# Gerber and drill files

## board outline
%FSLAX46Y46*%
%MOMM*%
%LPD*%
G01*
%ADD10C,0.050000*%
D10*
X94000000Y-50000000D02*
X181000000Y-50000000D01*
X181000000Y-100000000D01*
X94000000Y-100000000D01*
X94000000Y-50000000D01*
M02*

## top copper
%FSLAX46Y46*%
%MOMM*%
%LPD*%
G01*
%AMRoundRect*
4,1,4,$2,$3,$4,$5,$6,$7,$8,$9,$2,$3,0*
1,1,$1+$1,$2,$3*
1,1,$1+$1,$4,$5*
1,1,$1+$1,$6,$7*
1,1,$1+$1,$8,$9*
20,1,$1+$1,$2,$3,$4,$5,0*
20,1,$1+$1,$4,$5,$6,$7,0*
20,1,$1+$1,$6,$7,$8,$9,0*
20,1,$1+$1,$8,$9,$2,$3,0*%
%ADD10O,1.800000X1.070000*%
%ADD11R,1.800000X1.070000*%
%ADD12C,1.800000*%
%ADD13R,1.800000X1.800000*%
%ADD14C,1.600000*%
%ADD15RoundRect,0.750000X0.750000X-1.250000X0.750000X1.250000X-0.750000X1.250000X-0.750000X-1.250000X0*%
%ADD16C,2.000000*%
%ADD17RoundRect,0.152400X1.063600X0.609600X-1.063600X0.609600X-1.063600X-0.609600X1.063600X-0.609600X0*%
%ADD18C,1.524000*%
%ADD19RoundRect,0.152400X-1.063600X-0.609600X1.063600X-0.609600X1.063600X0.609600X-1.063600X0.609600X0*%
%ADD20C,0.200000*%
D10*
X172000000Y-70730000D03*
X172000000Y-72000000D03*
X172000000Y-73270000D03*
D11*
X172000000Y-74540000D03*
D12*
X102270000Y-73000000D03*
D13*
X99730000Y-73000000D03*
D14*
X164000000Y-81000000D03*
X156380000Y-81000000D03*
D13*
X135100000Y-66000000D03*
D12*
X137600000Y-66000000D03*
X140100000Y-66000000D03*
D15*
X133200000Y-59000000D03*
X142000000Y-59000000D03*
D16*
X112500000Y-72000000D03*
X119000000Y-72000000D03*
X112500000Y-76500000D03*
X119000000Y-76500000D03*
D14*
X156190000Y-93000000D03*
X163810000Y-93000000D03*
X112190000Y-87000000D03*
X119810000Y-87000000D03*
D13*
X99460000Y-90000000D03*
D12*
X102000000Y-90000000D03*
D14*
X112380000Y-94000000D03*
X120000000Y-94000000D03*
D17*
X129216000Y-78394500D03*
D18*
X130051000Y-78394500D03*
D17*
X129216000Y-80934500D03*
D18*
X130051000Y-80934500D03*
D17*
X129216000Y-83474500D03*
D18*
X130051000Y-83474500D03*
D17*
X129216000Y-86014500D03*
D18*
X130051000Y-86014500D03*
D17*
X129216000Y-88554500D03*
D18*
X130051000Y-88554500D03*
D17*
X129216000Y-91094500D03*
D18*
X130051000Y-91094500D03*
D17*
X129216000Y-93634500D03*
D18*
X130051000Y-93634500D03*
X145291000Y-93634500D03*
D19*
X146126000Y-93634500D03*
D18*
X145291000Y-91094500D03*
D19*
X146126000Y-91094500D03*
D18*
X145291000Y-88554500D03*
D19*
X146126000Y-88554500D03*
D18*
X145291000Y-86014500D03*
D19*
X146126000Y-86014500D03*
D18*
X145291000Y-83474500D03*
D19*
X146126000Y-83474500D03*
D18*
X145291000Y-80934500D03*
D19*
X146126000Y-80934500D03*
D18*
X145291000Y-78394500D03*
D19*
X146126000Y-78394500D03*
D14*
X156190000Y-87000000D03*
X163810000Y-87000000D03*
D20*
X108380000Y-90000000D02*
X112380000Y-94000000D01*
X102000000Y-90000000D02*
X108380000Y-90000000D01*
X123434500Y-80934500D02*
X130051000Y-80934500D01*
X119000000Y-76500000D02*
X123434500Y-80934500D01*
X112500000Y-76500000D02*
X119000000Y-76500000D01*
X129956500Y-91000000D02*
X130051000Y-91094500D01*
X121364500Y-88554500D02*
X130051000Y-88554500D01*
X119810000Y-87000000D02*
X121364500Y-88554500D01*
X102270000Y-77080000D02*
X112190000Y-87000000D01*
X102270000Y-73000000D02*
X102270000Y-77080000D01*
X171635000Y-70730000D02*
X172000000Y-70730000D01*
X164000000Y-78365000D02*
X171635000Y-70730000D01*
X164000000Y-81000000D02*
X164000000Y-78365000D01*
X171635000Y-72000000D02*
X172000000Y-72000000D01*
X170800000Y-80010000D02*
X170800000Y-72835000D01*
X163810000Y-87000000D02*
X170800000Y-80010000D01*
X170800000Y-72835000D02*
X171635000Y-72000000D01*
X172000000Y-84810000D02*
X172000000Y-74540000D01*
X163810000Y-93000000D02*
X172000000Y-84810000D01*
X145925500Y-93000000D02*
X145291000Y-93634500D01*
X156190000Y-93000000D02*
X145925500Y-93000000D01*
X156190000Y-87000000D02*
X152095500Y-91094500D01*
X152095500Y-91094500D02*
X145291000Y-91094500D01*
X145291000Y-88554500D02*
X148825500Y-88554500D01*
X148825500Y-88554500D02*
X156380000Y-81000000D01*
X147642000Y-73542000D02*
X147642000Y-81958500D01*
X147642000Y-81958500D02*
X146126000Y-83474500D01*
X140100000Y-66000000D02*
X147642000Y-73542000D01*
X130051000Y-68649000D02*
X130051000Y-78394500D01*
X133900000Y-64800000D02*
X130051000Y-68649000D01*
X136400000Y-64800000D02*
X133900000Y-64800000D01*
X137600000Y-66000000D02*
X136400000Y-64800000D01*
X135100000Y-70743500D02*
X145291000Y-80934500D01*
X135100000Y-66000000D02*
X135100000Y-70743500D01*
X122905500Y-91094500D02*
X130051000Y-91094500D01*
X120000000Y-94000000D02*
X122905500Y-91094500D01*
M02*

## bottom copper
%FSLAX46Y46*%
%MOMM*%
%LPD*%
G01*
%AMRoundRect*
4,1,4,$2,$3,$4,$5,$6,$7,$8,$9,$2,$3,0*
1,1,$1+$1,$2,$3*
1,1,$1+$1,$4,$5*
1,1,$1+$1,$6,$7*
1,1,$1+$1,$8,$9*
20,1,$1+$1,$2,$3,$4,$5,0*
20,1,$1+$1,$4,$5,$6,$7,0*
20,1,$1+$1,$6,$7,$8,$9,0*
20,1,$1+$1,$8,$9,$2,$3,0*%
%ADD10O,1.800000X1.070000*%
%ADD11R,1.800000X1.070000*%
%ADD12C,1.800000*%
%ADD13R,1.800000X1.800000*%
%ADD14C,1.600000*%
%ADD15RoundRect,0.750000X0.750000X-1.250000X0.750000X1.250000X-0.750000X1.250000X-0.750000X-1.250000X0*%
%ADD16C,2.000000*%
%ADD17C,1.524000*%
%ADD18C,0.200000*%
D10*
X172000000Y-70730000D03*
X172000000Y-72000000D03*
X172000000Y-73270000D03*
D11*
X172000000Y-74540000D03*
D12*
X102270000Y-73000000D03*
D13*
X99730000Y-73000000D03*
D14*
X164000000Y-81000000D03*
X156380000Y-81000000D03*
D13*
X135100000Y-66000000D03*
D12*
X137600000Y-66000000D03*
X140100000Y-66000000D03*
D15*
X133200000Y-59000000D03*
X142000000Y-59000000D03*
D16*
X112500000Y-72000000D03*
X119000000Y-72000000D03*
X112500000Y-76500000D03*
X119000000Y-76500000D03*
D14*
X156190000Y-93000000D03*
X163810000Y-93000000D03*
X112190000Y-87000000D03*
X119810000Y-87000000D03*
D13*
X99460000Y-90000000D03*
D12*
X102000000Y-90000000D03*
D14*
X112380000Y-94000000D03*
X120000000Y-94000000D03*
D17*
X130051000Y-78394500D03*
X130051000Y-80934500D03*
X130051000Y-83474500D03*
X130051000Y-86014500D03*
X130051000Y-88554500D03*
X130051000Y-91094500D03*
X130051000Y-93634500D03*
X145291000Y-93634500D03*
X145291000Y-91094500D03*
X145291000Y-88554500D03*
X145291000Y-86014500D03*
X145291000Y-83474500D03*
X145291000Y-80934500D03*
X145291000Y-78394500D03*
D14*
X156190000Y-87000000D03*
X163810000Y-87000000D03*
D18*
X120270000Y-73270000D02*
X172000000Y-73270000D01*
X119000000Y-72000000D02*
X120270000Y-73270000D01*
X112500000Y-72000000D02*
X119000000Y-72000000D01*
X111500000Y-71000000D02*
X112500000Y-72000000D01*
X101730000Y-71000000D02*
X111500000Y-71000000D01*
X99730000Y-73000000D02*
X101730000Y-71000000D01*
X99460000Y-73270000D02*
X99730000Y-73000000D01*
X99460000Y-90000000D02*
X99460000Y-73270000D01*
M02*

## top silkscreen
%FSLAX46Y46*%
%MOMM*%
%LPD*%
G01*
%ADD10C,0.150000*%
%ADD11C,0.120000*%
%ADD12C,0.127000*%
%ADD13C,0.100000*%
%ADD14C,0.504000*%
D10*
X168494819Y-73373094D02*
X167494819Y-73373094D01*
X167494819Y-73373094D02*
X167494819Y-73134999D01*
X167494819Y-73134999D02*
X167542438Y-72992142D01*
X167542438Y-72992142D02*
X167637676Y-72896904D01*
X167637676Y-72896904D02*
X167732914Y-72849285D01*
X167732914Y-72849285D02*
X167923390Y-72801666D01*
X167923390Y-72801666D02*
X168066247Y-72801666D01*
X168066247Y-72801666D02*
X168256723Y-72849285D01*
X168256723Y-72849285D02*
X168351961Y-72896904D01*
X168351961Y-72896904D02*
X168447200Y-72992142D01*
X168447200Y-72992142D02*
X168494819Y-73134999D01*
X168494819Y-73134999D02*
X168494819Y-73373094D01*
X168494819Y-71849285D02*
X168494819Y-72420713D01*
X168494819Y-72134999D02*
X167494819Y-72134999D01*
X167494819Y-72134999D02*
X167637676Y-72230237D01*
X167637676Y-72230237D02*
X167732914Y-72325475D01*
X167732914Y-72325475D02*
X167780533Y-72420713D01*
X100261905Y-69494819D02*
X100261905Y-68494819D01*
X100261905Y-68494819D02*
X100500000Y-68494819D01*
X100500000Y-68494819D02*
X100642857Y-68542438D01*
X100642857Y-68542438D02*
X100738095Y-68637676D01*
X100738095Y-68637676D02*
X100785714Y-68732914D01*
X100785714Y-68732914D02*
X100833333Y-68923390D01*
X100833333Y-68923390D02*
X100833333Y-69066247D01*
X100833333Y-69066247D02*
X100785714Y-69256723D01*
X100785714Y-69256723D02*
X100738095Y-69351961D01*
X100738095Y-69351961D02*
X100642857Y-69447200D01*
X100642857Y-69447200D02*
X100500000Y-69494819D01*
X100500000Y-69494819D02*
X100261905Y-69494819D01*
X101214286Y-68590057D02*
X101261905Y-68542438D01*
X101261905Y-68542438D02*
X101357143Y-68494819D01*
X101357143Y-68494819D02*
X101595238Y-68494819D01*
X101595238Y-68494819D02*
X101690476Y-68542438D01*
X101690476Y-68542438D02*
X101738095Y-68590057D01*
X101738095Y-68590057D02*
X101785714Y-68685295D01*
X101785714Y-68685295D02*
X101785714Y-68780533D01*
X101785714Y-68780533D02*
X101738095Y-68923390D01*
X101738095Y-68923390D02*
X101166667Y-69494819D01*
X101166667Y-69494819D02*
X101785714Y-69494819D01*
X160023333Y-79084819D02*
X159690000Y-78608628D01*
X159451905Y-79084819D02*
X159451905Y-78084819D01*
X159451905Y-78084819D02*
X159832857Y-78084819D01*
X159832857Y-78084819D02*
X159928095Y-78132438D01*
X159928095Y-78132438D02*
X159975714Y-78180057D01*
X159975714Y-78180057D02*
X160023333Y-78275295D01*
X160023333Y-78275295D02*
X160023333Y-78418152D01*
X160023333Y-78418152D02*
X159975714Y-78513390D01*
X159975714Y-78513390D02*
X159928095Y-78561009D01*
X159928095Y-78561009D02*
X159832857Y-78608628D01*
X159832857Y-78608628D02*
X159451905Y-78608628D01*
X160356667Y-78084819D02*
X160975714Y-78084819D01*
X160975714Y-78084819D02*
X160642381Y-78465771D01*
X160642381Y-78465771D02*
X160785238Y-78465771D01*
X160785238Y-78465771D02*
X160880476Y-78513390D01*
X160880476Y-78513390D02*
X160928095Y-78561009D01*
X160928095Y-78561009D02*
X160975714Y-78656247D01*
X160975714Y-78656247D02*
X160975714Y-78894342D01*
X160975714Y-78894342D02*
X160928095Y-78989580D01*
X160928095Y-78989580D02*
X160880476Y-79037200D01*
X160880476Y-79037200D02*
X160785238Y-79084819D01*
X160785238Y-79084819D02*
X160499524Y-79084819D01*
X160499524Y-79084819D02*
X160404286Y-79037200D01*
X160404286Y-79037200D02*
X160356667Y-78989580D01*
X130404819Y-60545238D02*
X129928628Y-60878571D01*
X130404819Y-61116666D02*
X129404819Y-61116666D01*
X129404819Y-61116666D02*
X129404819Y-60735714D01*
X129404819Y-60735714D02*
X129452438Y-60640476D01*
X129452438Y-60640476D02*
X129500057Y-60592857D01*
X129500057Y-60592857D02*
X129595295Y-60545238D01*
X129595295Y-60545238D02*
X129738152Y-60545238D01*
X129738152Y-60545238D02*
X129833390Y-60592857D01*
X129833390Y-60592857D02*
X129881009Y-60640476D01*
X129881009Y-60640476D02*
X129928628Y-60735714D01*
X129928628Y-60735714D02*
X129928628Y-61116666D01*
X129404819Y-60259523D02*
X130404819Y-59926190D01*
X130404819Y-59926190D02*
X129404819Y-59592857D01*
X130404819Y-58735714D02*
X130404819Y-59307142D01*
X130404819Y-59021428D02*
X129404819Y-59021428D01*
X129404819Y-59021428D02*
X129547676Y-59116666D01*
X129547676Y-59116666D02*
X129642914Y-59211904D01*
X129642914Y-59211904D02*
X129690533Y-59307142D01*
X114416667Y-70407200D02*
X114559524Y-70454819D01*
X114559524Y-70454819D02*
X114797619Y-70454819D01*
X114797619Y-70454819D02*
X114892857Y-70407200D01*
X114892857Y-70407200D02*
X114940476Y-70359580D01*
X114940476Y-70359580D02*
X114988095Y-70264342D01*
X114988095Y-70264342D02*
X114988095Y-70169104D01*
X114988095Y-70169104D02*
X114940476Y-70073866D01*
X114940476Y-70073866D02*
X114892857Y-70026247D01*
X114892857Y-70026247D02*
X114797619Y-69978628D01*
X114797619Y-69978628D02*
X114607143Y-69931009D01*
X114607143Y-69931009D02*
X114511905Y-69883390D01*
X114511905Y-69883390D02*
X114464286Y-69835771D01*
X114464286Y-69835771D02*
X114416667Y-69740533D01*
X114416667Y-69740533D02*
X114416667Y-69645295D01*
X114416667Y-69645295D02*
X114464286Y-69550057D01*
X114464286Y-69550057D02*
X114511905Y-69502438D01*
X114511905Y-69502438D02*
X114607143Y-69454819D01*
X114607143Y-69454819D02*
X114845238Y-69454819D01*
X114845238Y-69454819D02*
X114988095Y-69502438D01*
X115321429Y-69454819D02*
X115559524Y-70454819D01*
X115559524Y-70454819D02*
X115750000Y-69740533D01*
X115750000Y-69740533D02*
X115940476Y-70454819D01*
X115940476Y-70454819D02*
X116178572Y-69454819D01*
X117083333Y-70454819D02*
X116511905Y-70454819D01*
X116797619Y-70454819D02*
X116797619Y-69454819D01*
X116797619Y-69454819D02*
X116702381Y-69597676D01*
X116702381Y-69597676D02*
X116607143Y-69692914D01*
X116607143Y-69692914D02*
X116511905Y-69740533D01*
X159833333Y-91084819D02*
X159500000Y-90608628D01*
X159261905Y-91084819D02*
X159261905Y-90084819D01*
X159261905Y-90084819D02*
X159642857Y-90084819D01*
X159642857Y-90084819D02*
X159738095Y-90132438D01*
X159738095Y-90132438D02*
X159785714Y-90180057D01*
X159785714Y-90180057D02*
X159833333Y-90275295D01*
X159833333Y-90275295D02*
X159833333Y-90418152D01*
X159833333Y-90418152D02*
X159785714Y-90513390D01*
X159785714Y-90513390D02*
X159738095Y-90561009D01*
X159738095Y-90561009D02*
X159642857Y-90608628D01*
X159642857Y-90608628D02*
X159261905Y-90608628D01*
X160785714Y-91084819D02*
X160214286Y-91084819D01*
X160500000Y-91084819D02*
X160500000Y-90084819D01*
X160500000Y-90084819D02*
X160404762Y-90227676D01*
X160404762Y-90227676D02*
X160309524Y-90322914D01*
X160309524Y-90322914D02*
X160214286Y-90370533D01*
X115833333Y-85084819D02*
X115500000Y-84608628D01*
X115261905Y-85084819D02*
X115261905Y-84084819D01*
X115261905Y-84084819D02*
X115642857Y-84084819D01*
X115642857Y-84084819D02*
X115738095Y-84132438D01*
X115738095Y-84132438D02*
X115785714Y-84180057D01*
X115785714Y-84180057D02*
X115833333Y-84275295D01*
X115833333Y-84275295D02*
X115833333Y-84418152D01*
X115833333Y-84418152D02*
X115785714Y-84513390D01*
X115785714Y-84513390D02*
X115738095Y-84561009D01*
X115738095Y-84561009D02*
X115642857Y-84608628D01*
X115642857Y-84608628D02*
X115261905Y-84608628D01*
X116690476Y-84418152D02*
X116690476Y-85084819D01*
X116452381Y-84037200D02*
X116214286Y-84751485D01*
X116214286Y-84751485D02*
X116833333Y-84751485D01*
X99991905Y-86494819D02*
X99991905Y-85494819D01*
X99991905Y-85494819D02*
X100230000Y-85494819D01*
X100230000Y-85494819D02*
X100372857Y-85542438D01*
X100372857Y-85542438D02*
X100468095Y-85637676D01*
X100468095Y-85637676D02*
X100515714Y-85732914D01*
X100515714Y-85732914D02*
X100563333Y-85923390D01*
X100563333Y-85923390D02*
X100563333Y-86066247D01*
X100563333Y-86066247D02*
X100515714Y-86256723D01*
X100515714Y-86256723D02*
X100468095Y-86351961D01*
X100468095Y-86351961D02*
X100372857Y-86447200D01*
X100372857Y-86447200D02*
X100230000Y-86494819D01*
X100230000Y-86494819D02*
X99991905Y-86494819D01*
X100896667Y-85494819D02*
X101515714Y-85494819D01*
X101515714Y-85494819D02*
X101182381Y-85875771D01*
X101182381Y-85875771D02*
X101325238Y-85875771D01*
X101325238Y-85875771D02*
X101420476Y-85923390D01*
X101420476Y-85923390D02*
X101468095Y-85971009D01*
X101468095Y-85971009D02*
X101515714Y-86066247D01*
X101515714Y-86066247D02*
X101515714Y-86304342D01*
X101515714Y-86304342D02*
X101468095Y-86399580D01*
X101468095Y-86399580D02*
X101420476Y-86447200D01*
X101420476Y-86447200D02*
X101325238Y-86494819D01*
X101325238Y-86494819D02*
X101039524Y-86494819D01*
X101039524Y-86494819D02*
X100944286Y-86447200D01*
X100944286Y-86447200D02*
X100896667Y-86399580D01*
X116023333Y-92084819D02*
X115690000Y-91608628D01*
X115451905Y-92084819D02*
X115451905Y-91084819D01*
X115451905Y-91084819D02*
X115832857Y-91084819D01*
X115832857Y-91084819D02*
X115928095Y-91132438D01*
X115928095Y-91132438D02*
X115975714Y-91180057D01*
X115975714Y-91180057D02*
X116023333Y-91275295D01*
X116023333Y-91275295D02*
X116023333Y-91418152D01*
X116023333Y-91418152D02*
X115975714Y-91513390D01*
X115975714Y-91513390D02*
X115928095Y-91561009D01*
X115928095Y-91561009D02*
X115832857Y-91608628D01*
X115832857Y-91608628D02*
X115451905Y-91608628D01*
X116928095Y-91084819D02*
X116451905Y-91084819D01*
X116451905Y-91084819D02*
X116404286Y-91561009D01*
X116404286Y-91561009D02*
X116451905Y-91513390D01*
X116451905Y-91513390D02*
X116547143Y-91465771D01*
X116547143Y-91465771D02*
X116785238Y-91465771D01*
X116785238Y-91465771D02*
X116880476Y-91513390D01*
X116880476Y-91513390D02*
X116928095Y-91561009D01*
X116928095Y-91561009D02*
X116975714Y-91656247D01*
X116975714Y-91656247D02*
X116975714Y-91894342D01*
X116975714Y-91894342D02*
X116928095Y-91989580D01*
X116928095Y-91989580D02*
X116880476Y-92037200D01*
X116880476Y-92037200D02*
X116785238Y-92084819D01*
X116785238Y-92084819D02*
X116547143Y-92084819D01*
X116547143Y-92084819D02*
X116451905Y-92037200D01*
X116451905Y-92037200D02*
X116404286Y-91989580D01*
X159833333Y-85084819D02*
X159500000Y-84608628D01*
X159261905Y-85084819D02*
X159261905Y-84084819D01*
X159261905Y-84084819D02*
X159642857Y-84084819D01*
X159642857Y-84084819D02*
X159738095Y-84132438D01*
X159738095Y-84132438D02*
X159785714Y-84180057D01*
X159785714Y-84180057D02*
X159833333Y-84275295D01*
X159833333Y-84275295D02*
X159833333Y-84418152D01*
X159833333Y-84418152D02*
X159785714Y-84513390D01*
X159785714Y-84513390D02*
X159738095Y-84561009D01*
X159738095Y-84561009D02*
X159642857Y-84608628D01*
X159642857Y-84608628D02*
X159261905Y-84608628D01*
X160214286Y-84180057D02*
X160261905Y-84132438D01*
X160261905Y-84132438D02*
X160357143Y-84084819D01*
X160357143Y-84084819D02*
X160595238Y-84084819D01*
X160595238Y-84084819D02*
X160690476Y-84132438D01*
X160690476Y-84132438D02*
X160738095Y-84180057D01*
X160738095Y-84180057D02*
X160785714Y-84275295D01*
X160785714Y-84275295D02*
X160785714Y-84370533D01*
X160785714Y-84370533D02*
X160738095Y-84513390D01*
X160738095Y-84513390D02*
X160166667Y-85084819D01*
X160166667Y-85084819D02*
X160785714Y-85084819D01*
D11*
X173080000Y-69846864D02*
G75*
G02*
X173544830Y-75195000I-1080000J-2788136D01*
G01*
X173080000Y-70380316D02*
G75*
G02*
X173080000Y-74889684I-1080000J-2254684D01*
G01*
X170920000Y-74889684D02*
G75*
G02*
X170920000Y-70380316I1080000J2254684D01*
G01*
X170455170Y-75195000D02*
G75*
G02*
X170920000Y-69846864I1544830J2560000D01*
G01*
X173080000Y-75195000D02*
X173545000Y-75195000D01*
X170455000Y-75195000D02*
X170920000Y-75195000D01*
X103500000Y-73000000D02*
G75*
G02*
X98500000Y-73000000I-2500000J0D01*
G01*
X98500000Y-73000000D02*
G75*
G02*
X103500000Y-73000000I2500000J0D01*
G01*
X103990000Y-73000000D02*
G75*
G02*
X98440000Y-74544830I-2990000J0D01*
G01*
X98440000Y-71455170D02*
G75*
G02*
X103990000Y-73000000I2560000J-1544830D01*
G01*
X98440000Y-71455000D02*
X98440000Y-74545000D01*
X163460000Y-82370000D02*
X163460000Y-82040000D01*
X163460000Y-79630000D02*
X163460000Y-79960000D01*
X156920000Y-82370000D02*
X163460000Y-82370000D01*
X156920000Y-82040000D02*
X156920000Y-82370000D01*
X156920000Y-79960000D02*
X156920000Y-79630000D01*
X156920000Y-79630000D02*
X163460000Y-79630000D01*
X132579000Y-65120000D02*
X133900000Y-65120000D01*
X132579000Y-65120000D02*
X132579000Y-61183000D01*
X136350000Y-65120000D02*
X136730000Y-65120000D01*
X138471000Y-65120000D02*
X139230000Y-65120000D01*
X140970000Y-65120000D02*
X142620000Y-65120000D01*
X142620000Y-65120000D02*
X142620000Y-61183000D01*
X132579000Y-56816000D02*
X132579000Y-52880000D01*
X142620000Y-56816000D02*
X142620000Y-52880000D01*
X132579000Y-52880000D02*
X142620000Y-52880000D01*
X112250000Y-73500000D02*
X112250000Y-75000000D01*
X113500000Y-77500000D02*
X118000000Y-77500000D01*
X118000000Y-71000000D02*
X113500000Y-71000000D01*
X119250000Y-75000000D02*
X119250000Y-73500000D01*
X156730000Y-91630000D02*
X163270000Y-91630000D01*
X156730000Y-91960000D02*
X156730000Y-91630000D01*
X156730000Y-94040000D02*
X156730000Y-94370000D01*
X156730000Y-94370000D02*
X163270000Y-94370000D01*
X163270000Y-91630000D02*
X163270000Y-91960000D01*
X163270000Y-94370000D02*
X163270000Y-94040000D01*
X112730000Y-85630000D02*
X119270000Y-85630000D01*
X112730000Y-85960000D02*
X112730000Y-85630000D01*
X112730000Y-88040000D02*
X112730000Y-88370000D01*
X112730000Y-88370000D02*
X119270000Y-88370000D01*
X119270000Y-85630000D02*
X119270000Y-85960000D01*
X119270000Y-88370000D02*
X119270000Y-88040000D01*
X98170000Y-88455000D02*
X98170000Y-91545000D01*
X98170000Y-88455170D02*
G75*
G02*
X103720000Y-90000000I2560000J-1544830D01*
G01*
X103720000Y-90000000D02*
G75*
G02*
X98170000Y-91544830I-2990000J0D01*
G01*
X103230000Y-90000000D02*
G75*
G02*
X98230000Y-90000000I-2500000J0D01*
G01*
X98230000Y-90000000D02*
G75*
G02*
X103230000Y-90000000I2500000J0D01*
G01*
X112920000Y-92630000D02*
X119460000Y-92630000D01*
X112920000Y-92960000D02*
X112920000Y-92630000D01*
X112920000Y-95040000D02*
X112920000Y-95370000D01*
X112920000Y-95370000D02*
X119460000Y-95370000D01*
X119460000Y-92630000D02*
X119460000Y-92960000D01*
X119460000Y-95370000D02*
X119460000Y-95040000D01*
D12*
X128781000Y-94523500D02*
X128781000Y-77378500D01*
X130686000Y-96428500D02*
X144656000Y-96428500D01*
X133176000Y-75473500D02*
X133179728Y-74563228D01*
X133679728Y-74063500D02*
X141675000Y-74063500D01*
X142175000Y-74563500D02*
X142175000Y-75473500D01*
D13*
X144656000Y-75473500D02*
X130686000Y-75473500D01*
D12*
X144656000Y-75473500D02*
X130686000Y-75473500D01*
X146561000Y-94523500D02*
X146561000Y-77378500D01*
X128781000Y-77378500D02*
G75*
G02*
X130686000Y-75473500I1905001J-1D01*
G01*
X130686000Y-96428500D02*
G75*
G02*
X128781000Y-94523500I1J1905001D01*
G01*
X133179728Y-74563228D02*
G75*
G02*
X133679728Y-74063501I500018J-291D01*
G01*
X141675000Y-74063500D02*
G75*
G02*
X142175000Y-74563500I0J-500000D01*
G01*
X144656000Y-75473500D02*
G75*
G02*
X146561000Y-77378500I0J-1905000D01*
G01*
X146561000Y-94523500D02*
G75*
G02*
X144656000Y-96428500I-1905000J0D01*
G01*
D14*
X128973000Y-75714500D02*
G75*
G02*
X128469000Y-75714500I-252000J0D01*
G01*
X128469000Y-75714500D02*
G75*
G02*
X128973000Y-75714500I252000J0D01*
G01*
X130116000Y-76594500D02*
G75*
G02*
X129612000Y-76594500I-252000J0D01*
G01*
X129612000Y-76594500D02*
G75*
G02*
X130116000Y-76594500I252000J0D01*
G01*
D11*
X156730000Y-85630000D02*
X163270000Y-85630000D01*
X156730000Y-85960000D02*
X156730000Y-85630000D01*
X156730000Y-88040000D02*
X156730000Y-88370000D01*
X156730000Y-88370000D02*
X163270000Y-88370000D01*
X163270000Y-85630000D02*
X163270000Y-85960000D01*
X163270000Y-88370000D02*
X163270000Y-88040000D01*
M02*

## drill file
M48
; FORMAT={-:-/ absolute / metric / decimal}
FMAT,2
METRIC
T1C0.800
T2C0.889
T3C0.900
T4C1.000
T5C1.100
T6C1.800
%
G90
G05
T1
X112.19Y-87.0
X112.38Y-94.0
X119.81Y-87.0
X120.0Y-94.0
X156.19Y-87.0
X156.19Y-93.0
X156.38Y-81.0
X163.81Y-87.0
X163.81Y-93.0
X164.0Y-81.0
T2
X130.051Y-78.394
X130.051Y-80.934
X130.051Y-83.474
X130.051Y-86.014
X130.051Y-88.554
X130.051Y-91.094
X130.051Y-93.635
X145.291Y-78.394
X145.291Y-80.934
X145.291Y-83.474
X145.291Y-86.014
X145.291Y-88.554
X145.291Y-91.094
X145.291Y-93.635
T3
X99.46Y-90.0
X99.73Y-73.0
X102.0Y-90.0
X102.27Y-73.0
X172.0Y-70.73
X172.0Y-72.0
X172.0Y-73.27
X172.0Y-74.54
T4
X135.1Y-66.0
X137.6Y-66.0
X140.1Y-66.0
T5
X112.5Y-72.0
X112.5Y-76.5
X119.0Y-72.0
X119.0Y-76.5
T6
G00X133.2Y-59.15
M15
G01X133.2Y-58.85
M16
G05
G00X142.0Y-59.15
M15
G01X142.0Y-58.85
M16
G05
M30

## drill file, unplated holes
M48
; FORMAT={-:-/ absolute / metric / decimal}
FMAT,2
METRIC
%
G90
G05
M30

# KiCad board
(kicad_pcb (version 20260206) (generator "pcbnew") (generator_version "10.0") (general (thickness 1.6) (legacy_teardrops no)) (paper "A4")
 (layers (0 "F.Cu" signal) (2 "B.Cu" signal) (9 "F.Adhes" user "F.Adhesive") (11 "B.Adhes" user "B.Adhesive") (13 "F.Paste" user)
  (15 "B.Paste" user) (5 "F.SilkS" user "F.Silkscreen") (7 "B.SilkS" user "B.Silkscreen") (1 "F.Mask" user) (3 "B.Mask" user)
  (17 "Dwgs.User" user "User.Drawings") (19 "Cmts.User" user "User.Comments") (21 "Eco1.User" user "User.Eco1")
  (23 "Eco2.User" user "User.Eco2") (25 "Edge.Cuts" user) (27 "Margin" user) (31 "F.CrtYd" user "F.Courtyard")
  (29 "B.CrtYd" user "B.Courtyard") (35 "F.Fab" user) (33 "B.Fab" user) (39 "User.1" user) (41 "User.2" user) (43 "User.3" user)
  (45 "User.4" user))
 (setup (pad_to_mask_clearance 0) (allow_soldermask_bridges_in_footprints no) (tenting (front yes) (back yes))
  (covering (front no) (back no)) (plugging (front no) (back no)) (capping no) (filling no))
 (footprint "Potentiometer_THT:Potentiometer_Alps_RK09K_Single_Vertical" (layer "F.Cu") (at 135.1 66 90)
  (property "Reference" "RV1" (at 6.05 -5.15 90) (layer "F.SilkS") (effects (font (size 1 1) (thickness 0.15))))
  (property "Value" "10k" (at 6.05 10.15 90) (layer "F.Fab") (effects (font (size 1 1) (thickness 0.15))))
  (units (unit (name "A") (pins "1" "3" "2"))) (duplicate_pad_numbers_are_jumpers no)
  (fp_line (start 13.12 -2.521) (end 13.12 7.52) (stroke (width 0.12) (type solid)) (layer "F.SilkS"))
  (fp_line (start 9.184 -2.521) (end 13.12 -2.521) (stroke (width 0.12) (type solid)) (layer "F.SilkS"))
  (fp_line (start 0.88 -2.521) (end 4.817 -2.521) (stroke (width 0.12) (type solid)) (layer "F.SilkS"))
  (fp_line (start 0.88 -2.521) (end 0.88 -1.2) (stroke (width 0.12) (type solid)) (layer "F.SilkS"))
  (fp_line (start 0.88 1.25) (end 0.88 1.63) (stroke (width 0.12) (type solid)) (layer "F.SilkS"))
  (fp_line (start 0.88 3.371) (end 0.88 4.13) (stroke (width 0.12) (type solid)) (layer "F.SilkS"))
  (fp_line (start 0.88 5.87) (end 0.88 7.52) (stroke (width 0.12) (type solid)) (layer "F.SilkS"))
  (fp_line (start 9.184 7.52) (end 13.12 7.52) (stroke (width 0.12) (type solid)) (layer "F.SilkS"))
  (fp_line (start 0.88 7.52) (end 4.817 7.52) (stroke (width 0.12) (type solid)) (layer "F.SilkS"))
  (pad "1" thru_hole rect (at 0 0 90) (size 1.8 1.8) (drill 1) (layers "*.Cu" "*.Mask") (remove_unused_layers no) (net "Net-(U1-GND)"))
  (pad "2" thru_hole circle (at 0 2.5 90) (size 1.8 1.8) (drill 1) (layers "*.Cu" "*.Mask") (remove_unused_layers no)
   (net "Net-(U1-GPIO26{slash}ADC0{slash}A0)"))
  (pad "3" thru_hole circle (at 0 5 90) (size 1.8 1.8) (drill 1) (layers "*.Cu" "*.Mask") (remove_unused_layers no) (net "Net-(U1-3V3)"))
  (pad "MP" thru_hole roundrect (at 7 -1.9 90) (size 4 3) (drill oval 2.1 1.8) (layers "*.Cu" "*.Mask") (remove_unused_layers no)
   (roundrect_rratio 0.25))
  (pad "MP" thru_hole roundrect (at 7 6.9 90) (size 4 3) (drill oval 2.1 1.8) (layers "*.Cu" "*.Mask") (remove_unused_layers no)
   (roundrect_rratio 0.25)))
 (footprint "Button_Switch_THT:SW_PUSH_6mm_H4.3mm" (layer "F.Cu") (at 112.5 72)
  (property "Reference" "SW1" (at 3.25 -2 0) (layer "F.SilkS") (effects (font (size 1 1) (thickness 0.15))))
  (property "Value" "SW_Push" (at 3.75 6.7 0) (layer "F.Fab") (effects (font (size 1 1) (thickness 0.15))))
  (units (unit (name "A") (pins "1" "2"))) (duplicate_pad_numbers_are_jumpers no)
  (fp_line (start -0.25 1.5) (end -0.25 3) (stroke (width 0.12) (type solid)) (layer "F.SilkS"))
  (fp_line (start 1 5.5) (end 5.5 5.5) (stroke (width 0.12) (type solid)) (layer "F.SilkS"))
  (fp_line (start 5.5 -1) (end 1 -1) (stroke (width 0.12) (type solid)) (layer "F.SilkS"))
  (fp_line (start 6.75 3) (end 6.75 1.5) (stroke (width 0.12) (type solid)) (layer "F.SilkS"))
  (pad "1" thru_hole circle (at 0 0 90) (size 2 2) (drill 1.1) (layers "*.Cu" "*.Mask") (remove_unused_layers no) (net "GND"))
  (pad "1" thru_hole circle (at 6.5 0 90) (size 2 2) (drill 1.1) (layers "*.Cu" "*.Mask") (remove_unused_layers no) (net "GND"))
  (pad "2" thru_hole circle (at 0 4.5 90) (size 2 2) (drill 1.1) (layers "*.Cu" "*.Mask") (remove_unused_layers no)
   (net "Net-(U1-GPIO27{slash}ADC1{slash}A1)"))
  (pad "2" thru_hole circle (at 6.5 4.5 90) (size 2 2) (drill 1.1) (layers "*.Cu" "*.Mask") (remove_unused_layers no)
   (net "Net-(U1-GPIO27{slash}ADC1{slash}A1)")))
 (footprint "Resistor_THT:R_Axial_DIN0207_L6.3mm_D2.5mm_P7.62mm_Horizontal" (layer "F.Cu") (at 156.38 81)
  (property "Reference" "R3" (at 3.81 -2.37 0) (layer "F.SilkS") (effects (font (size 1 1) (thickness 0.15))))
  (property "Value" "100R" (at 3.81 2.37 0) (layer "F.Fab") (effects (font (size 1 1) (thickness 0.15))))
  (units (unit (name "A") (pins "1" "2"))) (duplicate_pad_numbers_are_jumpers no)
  (fp_line (start 0.54 -1.37) (end 7.08 -1.37) (stroke (width 0.12) (type solid)) (layer "F.SilkS"))
  (fp_line (start 0.54 -1.04) (end 0.54 -1.37) (stroke (width 0.12) (type solid)) (layer "F.SilkS"))
  (fp_line (start 0.54 1.04) (end 0.54 1.37) (stroke (width 0.12) (type solid)) (layer "F.SilkS"))
  (fp_line (start 0.54 1.37) (end 7.08 1.37) (stroke (width 0.12) (type solid)) (layer "F.SilkS"))
  (fp_line (start 7.08 -1.37) (end 7.08 -1.04) (stroke (width 0.12) (type solid)) (layer "F.SilkS"))
  (fp_line (start 7.08 1.37) (end 7.08 1.04) (stroke (width 0.12) (type solid)) (layer "F.SilkS"))
  (pad "1" thru_hole circle (at 0 0) (size 1.6 1.6) (drill 0.8) (layers "*.Cu" "*.Mask") (remove_unused_layers no)
   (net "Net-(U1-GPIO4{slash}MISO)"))
  (pad "2" thru_hole circle (at 7.62 0) (size 1.6 1.6) (drill 0.8) (layers "*.Cu" "*.Mask") (remove_unused_layers no) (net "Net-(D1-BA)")))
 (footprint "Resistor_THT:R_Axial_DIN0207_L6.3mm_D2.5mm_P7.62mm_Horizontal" (layer "F.Cu") (at 156.19 93)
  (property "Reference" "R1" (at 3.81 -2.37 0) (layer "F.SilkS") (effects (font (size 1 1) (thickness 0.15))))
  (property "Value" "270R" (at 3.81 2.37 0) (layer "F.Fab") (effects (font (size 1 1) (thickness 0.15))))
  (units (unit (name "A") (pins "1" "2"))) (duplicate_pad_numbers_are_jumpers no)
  (fp_line (start 0.54 -1.37) (end 7.08 -1.37) (stroke (width 0.12) (type solid)) (layer "F.SilkS"))
  (fp_line (start 0.54 -1.04) (end 0.54 -1.37) (stroke (width 0.12) (type solid)) (layer "F.SilkS"))
  (fp_line (start 0.54 1.04) (end 0.54 1.37) (stroke (width 0.12) (type solid)) (layer "F.SilkS"))
  (fp_line (start 0.54 1.37) (end 7.08 1.37) (stroke (width 0.12) (type solid)) (layer "F.SilkS"))
  (fp_line (start 7.08 -1.37) (end 7.08 -1.04) (stroke (width 0.12) (type solid)) (layer "F.SilkS"))
  (fp_line (start 7.08 1.37) (end 7.08 1.04) (stroke (width 0.12) (type solid)) (layer "F.SilkS"))
  (pad "1" thru_hole circle (at 0 0) (size 1.6 1.6) (drill 0.8) (layers "*.Cu" "*.Mask") (remove_unused_layers no)
   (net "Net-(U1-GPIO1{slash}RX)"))
  (pad "2" thru_hole circle (at 7.62 0) (size 1.6 1.6) (drill 0.8) (layers "*.Cu" "*.Mask") (remove_unused_layers no) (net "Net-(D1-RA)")))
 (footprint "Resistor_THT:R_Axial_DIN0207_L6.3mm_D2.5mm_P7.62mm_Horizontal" (layer "F.Cu") (at 112.19 87)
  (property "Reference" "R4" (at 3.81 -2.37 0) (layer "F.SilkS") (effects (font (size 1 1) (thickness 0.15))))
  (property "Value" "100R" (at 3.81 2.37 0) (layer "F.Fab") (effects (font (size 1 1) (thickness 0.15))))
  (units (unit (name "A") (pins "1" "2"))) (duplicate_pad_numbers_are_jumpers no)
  (fp_line (start 0.54 -1.37) (end 7.08 -1.37) (stroke (width 0.12) (type solid)) (layer "F.SilkS"))
  (fp_line (start 0.54 -1.04) (end 0.54 -1.37) (stroke (width 0.12) (type solid)) (layer "F.SilkS"))
  (fp_line (start 0.54 1.04) (end 0.54 1.37) (stroke (width 0.12) (type solid)) (layer "F.SilkS"))
  (fp_line (start 0.54 1.37) (end 7.08 1.37) (stroke (width 0.12) (type solid)) (layer "F.SilkS"))
  (fp_line (start 7.08 -1.37) (end 7.08 -1.04) (stroke (width 0.12) (type solid)) (layer "F.SilkS"))
  (fp_line (start 7.08 1.37) (end 7.08 1.04) (stroke (width 0.12) (type solid)) (layer "F.SilkS"))
  (pad "1" thru_hole circle (at 0 0) (size 1.6 1.6) (drill 0.8) (layers "*.Cu" "*.Mask") (remove_unused_layers no) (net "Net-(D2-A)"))
  (pad "2" thru_hole circle (at 7.62 0) (size 1.6 1.6) (drill 0.8) (layers "*.Cu" "*.Mask") (remove_unused_layers no)
   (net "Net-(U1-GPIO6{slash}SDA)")))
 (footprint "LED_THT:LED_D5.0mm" (layer "F.Cu") (at 99.46 90)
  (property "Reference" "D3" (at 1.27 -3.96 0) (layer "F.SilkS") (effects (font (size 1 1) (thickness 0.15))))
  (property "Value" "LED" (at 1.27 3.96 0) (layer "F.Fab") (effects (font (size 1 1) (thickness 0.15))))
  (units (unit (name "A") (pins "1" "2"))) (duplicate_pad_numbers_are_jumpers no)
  (fp_line (start -1.29 -1.545) (end -1.29 1.545) (stroke (width 0.12) (type solid)) (layer "F.SilkS"))
  (fp_arc (start -1.29 -1.54483) (mid 2.071779 -2.880495) (end 4.26 0) (stroke (width 0.12) (type solid)) (layer "F.SilkS"))
  (fp_arc (start 4.26 0) (mid 2.071779 2.880495) (end -1.29 1.54483) (stroke (width 0.12) (type solid)) (layer "F.SilkS"))
  (fp_circle (center 1.27 0) (end 3.77 0) (stroke (width 0.12) (type solid)) (fill no) (layer "F.SilkS"))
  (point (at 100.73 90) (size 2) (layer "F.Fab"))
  (pad "1" thru_hole rect (at 0 0) (size 1.8 1.8) (drill 0.9) (layers "*.Cu" "*.Mask") (remove_unused_layers no) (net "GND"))
  (pad "2" thru_hole circle (at 2.54 0) (size 1.8 1.8) (drill 0.9) (layers "*.Cu" "*.Mask") (remove_unused_layers no) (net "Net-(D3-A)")))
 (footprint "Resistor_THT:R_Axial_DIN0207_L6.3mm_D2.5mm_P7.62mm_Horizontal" (layer "F.Cu") (at 112.38 94)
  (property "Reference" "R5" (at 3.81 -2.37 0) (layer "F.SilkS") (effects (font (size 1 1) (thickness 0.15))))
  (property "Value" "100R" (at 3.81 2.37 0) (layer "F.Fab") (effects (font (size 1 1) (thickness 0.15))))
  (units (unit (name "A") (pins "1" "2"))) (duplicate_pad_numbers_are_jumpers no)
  (fp_line (start 0.54 -1.37) (end 7.08 -1.37) (stroke (width 0.12) (type solid)) (layer "F.SilkS"))
  (fp_line (start 0.54 -1.04) (end 0.54 -1.37) (stroke (width 0.12) (type solid)) (layer "F.SilkS"))
  (fp_line (start 0.54 1.04) (end 0.54 1.37) (stroke (width 0.12) (type solid)) (layer "F.SilkS"))
  (fp_line (start 0.54 1.37) (end 7.08 1.37) (stroke (width 0.12) (type solid)) (layer "F.SilkS"))
  (fp_line (start 7.08 -1.37) (end 7.08 -1.04) (stroke (width 0.12) (type solid)) (layer "F.SilkS"))
  (fp_line (start 7.08 1.37) (end 7.08 1.04) (stroke (width 0.12) (type solid)) (layer "F.SilkS"))
  (pad "1" thru_hole circle (at 0 0) (size 1.6 1.6) (drill 0.8) (layers "*.Cu" "*.Mask") (remove_unused_layers no) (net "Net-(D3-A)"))
  (pad "2" thru_hole circle (at 7.62 0) (size 1.6 1.6) (drill 0.8) (layers "*.Cu" "*.Mask") (remove_unused_layers no)
   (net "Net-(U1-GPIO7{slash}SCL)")))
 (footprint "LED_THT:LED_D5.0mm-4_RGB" (layer "F.Cu") (at 172 74.54 90)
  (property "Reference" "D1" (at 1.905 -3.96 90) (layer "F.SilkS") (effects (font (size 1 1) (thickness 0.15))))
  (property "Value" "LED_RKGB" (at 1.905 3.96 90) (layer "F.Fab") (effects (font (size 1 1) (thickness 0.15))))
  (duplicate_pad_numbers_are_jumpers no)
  (fp_line (start -0.655 -1.545) (end -0.655 -1.08) (stroke (width 0.12) (type solid)) (layer "F.SilkS"))
  (fp_line (start -0.655 1.08) (end -0.655 1.545) (stroke (width 0.12) (type solid)) (layer "F.SilkS"))
  (fp_arc (start -0.655 -1.54483) (mid 2.163898 -2.97877) (end 4.693136 -1.08) (stroke (width 0.12) (type solid)) (layer "F.SilkS"))
  (fp_arc (start -0.349684 -1.08) (mid 1.905 -2.5) (end 4.159684 -1.08) (stroke (width 0.12) (type solid)) (layer "F.SilkS"))
  (fp_arc (start 4.693136 1.08) (mid 2.163898 2.97877) (end -0.655 1.54483) (stroke (width 0.12) (type solid)) (layer "F.SilkS"))
  (fp_arc (start 4.159684 1.08) (mid 1.905 2.5) (end -0.349684 1.08) (stroke (width 0.12) (type solid)) (layer "F.SilkS"))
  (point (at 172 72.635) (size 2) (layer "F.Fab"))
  (pad "1" thru_hole rect (at 0 0 90) (size 1.07 1.8) (drill 0.9) (layers "*.Cu" "*.Mask") (remove_unused_layers no) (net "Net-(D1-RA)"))
  (pad "2" thru_hole oval (at 1.27 0 90) (size 1.07 1.8) (drill 0.9) (layers "*.Cu" "*.Mask") (remove_unused_layers no) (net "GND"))
  (pad "3" thru_hole oval (at 2.54 0 90) (size 1.07 1.8) (drill 0.9) (layers "*.Cu" "*.Mask") (remove_unused_layers no) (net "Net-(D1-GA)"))
  (pad "4" thru_hole oval (at 3.81 0 90) (size 1.07 1.8) (drill 0.9) (layers "*.Cu" "*.Mask") (remove_unused_layers no) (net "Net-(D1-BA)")))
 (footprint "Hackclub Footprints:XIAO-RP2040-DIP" (layer "F.Cu") (at 137.671 86.0145)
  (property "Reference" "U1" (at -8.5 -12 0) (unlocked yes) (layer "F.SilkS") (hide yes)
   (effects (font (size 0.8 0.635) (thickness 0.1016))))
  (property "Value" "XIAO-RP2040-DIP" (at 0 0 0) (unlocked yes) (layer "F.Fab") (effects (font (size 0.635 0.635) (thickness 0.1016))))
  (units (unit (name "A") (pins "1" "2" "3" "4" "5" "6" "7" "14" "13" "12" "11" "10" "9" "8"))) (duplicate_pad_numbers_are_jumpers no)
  (fp_line (start -8.89 8.509) (end -8.89 -8.636) (stroke (width 0.127) (type solid)) (layer "F.SilkS"))
  (fp_line (start -6.985 10.414) (end 6.985 10.414) (stroke (width 0.127) (type solid)) (layer "F.SilkS"))
  (fp_line (start -4.495 -10.541) (end -4.491272 -11.451272) (stroke (width 0.127) (type solid)) (layer "F.SilkS"))
  (fp_line (start -3.991272 -11.951) (end 4.004 -11.951) (stroke (width 0.127) (type solid)) (layer "F.SilkS"))
  (fp_line (start 4.504 -11.451) (end 4.504 -10.541) (stroke (width 0.127) (type solid)) (layer "F.SilkS"))
  (fp_line (start 6.985 -10.541) (end -6.985 -10.541) (stroke (width 0.1) (type solid)) (layer "F.SilkS"))
  (fp_line (start 6.985 -10.541) (end -6.985 -10.541) (stroke (width 0.127) (type solid)) (layer "F.SilkS"))
  (fp_line (start 8.89 8.509) (end 8.89 -8.636) (stroke (width 0.127) (type solid)) (layer "F.SilkS"))
  (fp_arc (start -8.89 -8.636) (mid -8.332038 -9.983038) (end -6.985 -10.541) (stroke (width 0.127) (type solid)) (layer "F.SilkS"))
  (fp_arc (start -6.985 10.414) (mid -8.332038 9.856038) (end -8.89 8.509) (stroke (width 0.127) (type solid)) (layer "F.SilkS"))
  (fp_arc (start -4.491272 -11.451272) (mid -4.344728 -11.80464) (end -3.991272 -11.951) (stroke (width 0.127) (type default))
   (layer "F.SilkS"))
  (fp_arc (start 4.004 -11.951) (mid 4.357553 -11.804553) (end 4.504 -11.451) (stroke (width 0.127) (type default)) (layer "F.SilkS"))
  (fp_arc (start 6.985 -10.541) (mid 8.332038 -9.983038) (end 8.89 -8.636) (stroke (width 0.127) (type solid)) (layer "F.SilkS"))
  (fp_arc (start 8.89 8.509) (mid 8.332038 9.856038) (end 6.985 10.414) (stroke (width 0.127) (type solid)) (layer "F.SilkS"))
  (fp_circle (center -8.95 -10.3) (end -8.95 -10.554) (stroke (width 0.5) (type solid)) (fill yes) (layer "F.SilkS"))
  (fp_circle (center -7.807 -9.42) (end -7.807 -9.674) (stroke (width 0.5) (type solid)) (fill yes) (layer "F.SilkS"))
  (pad "1" smd roundrect (at -8.455 -7.62 180) (size 2.432 1.524) (layers "F.Cu" "F.Mask") (roundrect_rratio 0.1)
   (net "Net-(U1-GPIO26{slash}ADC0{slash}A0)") (thermal_bridge_angle 45))
  (pad "1" thru_hole circle (at -7.62 -7.62 180) (size 1.524 1.524) (drill 0.889) (layers "*.Cu" "*.Mask") (remove_unused_layers no)
   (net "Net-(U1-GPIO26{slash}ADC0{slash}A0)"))
  (pad "2" smd roundrect (at -8.455 -5.08 180) (size 2.432 1.524) (layers "F.Cu" "F.Mask") (roundrect_rratio 0.1)
   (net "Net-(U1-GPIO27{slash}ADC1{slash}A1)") (thermal_bridge_angle 45))
  (pad "2" thru_hole circle (at -7.62 -5.08 180) (size 1.524 1.524) (drill 0.889) (layers "*.Cu" "*.Mask") (remove_unused_layers no)
   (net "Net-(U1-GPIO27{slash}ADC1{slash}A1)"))
  (pad "3" smd roundrect (at -8.455 -2.54 180) (size 2.432 1.524) (layers "F.Cu" "F.Mask") (roundrect_rratio 0.1)
   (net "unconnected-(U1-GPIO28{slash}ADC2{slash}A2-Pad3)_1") (thermal_bridge_angle 45))
  (pad "3" thru_hole circle (at -7.62 -2.54 180) (size 1.524 1.524) (drill 0.889) (layers "*.Cu" "*.Mask") (remove_unused_layers no)
   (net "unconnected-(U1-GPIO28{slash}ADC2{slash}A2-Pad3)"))
  (pad "4" smd roundrect (at -8.455 0 180) (size 2.432 1.524) (layers "F.Cu" "F.Mask") (roundrect_rratio 0.1)
   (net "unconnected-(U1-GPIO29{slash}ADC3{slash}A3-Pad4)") (thermal_bridge_angle 45))
  (pad "4" thru_hole circle (at -7.62 0 180) (size 1.524 1.524) (drill 0.889) (layers "*.Cu" "*.Mask") (remove_unused_layers no)
   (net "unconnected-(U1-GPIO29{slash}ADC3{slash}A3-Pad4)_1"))
  (pad "5" smd roundrect (at -8.455 2.54 180) (size 2.432 1.524) (layers "F.Cu" "F.Mask") (roundrect_rratio 0.1)
   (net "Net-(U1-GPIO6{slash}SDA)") (thermal_bridge_angle 45))
  (pad "5" thru_hole circle (at -7.62 2.54 180) (size 1.524 1.524) (drill 0.889) (layers "*.Cu" "*.Mask") (remove_unused_layers no)
   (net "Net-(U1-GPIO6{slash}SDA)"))
  (pad "6" smd roundrect (at -8.455 5.08 180) (size 2.432 1.524) (layers "F.Cu" "F.Mask") (roundrect_rratio 0.1)
   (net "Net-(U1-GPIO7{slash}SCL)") (thermal_bridge_angle 45))
  (pad "6" thru_hole circle (at -7.62 5.08 180) (size 1.524 1.524) (drill 0.889) (layers "*.Cu" "*.Mask") (remove_unused_layers no)
   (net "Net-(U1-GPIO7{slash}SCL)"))
  (pad "7" smd roundrect (at -8.455 7.62 180) (size 2.432 1.524) (layers "F.Cu" "F.Mask") (roundrect_rratio 0.1)
   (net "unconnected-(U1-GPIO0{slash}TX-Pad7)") (thermal_bridge_angle 45))
  (pad "7" thru_hole circle (at -7.62 7.62 180) (size 1.524 1.524) (drill 0.889) (layers "*.Cu" "*.Mask") (remove_unused_layers no)
   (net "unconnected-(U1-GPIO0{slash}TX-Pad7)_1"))
  (pad "8" thru_hole circle (at 7.62 7.62) (size 1.524 1.524) (drill 0.889) (layers "*.Cu" "*.Mask") (remove_unused_layers no)
   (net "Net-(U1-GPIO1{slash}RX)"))
  (pad "8" smd roundrect (at 8.455 7.62) (size 2.432 1.524) (layers "F.Cu" "F.Mask") (roundrect_rratio 0.1) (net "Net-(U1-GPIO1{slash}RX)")
   (thermal_bridge_angle 45))
  (pad "9" thru_hole circle (at 7.62 5.08) (size 1.524 1.524) (drill 0.889) (layers "*.Cu" "*.Mask") (remove_unused_layers no)
   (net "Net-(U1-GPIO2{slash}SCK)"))
  (pad "9" smd roundrect (at 8.455 5.08) (size 2.432 1.524) (layers "F.Cu" "F.Mask") (roundrect_rratio 0.1) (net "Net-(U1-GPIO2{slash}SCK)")
   (thermal_bridge_angle 45))
  (pad "10" thru_hole circle (at 7.62 2.54) (size 1.524 1.524) (drill 0.889) (layers "*.Cu" "*.Mask") (remove_unused_layers no)
   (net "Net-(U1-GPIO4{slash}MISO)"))
  (pad "10" smd roundrect (at 8.455 2.54) (size 2.432 1.524) (layers "F.Cu" "F.Mask") (roundrect_rratio 0.1)
   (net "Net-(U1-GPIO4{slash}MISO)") (thermal_bridge_angle 45))
  (pad "11" thru_hole circle (at 7.62 0) (size 1.524 1.524) (drill 0.889) (layers "*.Cu" "*.Mask") (remove_unused_layers no)
   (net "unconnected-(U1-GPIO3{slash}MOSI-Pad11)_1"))
  (pad "11" smd roundrect (at 8.455 0) (size 2.432 1.524) (layers "F.Cu" "F.Mask") (roundrect_rratio 0.1)
   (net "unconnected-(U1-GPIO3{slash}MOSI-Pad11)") (thermal_bridge_angle 45))
  (pad "12" thru_hole circle (at 7.62 -2.54) (size 1.524 1.524) (drill 0.889) (layers "*.Cu" "*.Mask") (remove_unused_layers no)
   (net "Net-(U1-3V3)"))
  (pad "12" smd roundrect (at 8.455 -2.54) (size 2.432 1.524) (layers "F.Cu" "F.Mask") (roundrect_rratio 0.1) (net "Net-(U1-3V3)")
   (thermal_bridge_angle 45))
  (pad "13" thru_hole circle (at 7.62 -5.08) (size 1.524 1.524) (drill 0.889) (layers "*.Cu" "*.Mask") (remove_unused_layers no)
   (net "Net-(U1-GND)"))
  (pad "13" smd roundrect (at 8.455 -5.08) (size 2.432 1.524) (layers "F.Cu" "F.Mask") (roundrect_rratio 0.1) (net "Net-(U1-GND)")
   (thermal_bridge_angle 45))
  (pad "14" thru_hole circle (at 7.62 -7.62) (size 1.524 1.524) (drill 0.889) (layers "*.Cu" "*.Mask") (remove_unused_layers no)
   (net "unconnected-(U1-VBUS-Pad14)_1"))
  (pad "14" smd roundrect (at 8.455 -7.62) (size 2.432 1.524) (layers "F.Cu" "F.Mask") (roundrect_rratio 0.1)
   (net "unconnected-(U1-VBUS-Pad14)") (thermal_bridge_angle 45)))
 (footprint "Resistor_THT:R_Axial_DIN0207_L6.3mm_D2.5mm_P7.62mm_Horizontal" (layer "F.Cu") (at 156.19 87)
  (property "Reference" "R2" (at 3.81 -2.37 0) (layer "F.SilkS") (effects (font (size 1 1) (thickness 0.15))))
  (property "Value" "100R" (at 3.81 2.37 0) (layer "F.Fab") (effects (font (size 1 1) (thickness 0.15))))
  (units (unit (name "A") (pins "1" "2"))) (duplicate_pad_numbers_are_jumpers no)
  (fp_line (start 0.54 -1.37) (end 7.08 -1.37) (stroke (width 0.12) (type solid)) (layer "F.SilkS"))
  (fp_line (start 0.54 -1.04) (end 0.54 -1.37) (stroke (width 0.12) (type solid)) (layer "F.SilkS"))
  (fp_line (start 0.54 1.04) (end 0.54 1.37) (stroke (width 0.12) (type solid)) (layer "F.SilkS"))
  (fp_line (start 0.54 1.37) (end 7.08 1.37) (stroke (width 0.12) (type solid)) (layer "F.SilkS"))
  (fp_line (start 7.08 -1.37) (end 7.08 -1.04) (stroke (width 0.12) (type solid)) (layer "F.SilkS"))
  (fp_line (start 7.08 1.37) (end 7.08 1.04) (stroke (width 0.12) (type solid)) (layer "F.SilkS"))
  (pad "1" thru_hole circle (at 0 0) (size 1.6 1.6) (drill 0.8) (layers "*.Cu" "*.Mask") (remove_unused_layers no)
   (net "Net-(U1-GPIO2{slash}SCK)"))
  (pad "2" thru_hole circle (at 7.62 0) (size 1.6 1.6) (drill 0.8) (layers "*.Cu" "*.Mask") (remove_unused_layers no) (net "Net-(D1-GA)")))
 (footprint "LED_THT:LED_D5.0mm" (layer "F.Cu") (at 99.73 73)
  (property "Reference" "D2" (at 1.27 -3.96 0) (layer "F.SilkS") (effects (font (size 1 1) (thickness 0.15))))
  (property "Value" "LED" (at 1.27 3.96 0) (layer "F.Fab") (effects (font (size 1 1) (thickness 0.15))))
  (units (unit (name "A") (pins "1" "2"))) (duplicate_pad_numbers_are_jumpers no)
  (fp_line (start -1.29 -1.545) (end -1.29 1.545) (stroke (width 0.12) (type solid)) (layer "F.SilkS"))
  (fp_arc (start -1.29 -1.54483) (mid 2.071779 -2.880495) (end 4.26 0) (stroke (width 0.12) (type solid)) (layer "F.SilkS"))
  (fp_arc (start 4.26 0) (mid 2.071779 2.880495) (end -1.29 1.54483) (stroke (width 0.12) (type solid)) (layer "F.SilkS"))
  (fp_circle (center 1.27 0) (end 3.77 0) (stroke (width 0.12) (type solid)) (fill no) (layer "F.SilkS"))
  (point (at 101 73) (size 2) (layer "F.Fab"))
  (pad "1" thru_hole rect (at 0 0) (size 1.8 1.8) (drill 0.9) (layers "*.Cu" "*.Mask") (remove_unused_layers no) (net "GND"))
  (pad "2" thru_hole circle (at 2.54 0) (size 1.8 1.8) (drill 0.9) (layers "*.Cu" "*.Mask") (remove_unused_layers no) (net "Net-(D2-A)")))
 (gr_rect (start 94 50) (end 181 100) (stroke (width 0.05) (type default)) (fill no) (layer "Edge.Cuts"))
 (segment (start 135.1 66) (end 135.1 70.7435) (width 0.2) (layer "F.Cu") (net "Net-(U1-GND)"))
 (segment (start 135.1 70.7435) (end 145.291 80.9345) (width 0.2) (layer "F.Cu") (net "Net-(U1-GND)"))
 (segment (start 133.9 64.8) (end 130.051 68.649) (width 0.2) (layer "F.Cu") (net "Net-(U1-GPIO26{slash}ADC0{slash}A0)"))
 (segment (start 137.6 66) (end 136.4 64.8) (width 0.2) (layer "F.Cu") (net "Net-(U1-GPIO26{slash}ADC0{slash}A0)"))
 (segment (start 136.4 64.8) (end 133.9 64.8) (width 0.2) (layer "F.Cu") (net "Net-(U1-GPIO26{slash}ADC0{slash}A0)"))
 (segment (start 130.051 68.649) (end 130.051 78.3945) (width 0.2) (layer "F.Cu") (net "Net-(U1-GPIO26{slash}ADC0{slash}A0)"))
 (segment (start 140.1 66) (end 147.642 73.542) (width 0.2) (layer "F.Cu") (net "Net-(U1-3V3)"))
 (segment (start 147.642 73.542) (end 147.642 81.9585) (width 0.2) (layer "F.Cu") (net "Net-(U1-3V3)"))
 (segment (start 147.642 81.9585) (end 146.126 83.4745) (width 0.2) (layer "F.Cu") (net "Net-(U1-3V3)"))
 (segment (start 111.5 71) (end 112.5 72) (width 0.2) (layer "B.Cu") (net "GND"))
 (segment (start 101.73 71) (end 111.5 71) (width 0.2) (layer "B.Cu") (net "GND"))
 (segment (start 99.73 73) (end 101.73 71) (width 0.2) (layer "B.Cu") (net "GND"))
 (segment (start 119 72) (end 120.27 73.27) (width 0.2) (layer "B.Cu") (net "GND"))
 (segment (start 99.46 90) (end 99.46 73.27) (width 0.2) (layer "B.Cu") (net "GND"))
 (segment (start 112.5 72) (end 119 72) (width 0.2) (layer "B.Cu") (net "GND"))
 (segment (start 120.27 73.27) (end 172 73.27) (width 0.2) (layer "B.Cu") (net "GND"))
 (segment (start 99.46 73.27) (end 99.73 73) (width 0.2) (layer "B.Cu") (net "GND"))
 (segment (start 119 76.5) (end 123.4345 80.9345) (width 0.2) (layer "F.Cu") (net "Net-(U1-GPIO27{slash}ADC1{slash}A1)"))
 (segment (start 112.5 76.5) (end 119 76.5) (width 0.2) (layer "F.Cu") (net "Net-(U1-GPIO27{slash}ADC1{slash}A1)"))
 (segment (start 123.4345 80.9345) (end 130.051 80.9345) (width 0.2) (layer "F.Cu") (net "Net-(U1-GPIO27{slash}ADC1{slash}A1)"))
 (segment (start 145.291 88.5545) (end 148.8255 88.5545) (width 0.2) (layer "F.Cu") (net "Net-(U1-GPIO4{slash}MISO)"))
 (segment (start 148.8255 88.5545) (end 156.38 81) (width 0.2) (layer "F.Cu") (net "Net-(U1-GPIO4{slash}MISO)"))
 (segment (start 164 81) (end 164 78.365) (width 0.2) (layer "F.Cu") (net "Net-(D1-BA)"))
 (segment (start 171.635 70.73) (end 172 70.73) (width 0.2) (layer "F.Cu") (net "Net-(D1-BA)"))
 (segment (start 164 78.365) (end 171.635 70.73) (width 0.2) (layer "F.Cu") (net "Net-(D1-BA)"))
 (segment (start 145.9255 93) (end 145.291 93.6345) (width 0.2) (layer "F.Cu") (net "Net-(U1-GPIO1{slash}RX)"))
 (segment (start 156.19 93) (end 145.9255 93) (width 0.2) (layer "F.Cu") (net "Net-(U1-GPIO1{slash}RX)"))
 (segment (start 163.81 93) (end 172 84.81) (width 0.2) (layer "F.Cu") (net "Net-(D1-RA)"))
 (segment (start 172 84.81) (end 172 74.54) (width 0.2) (layer "F.Cu") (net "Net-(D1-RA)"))
 (segment (start 102.27 77.08) (end 112.19 87) (width 0.2) (layer "F.Cu") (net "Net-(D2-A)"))
 (segment (start 102.27 73) (end 102.27 77.08) (width 0.2) (layer "F.Cu") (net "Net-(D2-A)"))
 (segment (start 121.3645 88.5545) (end 130.051 88.5545) (width 0.2) (layer "F.Cu") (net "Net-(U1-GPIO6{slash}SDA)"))
 (segment (start 119.81 87) (end 121.3645 88.5545) (width 0.2) (layer "F.Cu") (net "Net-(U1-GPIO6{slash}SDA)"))
 (segment (start 102 90) (end 108.38 90) (width 0.2) (layer "F.Cu") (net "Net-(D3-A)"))
 (segment (start 108.38 90) (end 112.38 94) (width 0.2) (layer "F.Cu") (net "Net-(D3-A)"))
 (segment (start 129.9565 91) (end 130.051 91.0945) (width 0.2) (layer "F.Cu") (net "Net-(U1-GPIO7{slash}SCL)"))
 (segment (start 120 94) (end 122.9055 91.0945) (width 0.2) (layer "F.Cu") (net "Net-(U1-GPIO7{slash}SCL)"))
 (segment (start 122.9055 91.0945) (end 130.051 91.0945) (width 0.2) (layer "F.Cu") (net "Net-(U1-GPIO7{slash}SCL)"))
 (segment (start 163.81 87) (end 170.8 80.01) (width 0.2) (layer "F.Cu") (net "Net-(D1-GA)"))
 (segment (start 170.8 72.835) (end 171.635 72) (width 0.2) (layer "F.Cu") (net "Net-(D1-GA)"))
 (segment (start 171.635 72) (end 172 72) (width 0.2) (layer "F.Cu") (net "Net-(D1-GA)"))
 (segment (start 170.8 80.01) (end 170.8 72.835) (width 0.2) (layer "F.Cu") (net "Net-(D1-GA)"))
 (segment (start 152.0955 91.0945) (end 145.291 91.0945) (width 0.2) (layer "F.Cu") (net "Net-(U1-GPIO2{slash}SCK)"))
 (segment (start 156.19 87) (end 152.0955 91.0945) (width 0.2) (layer "F.Cu") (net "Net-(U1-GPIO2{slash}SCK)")))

